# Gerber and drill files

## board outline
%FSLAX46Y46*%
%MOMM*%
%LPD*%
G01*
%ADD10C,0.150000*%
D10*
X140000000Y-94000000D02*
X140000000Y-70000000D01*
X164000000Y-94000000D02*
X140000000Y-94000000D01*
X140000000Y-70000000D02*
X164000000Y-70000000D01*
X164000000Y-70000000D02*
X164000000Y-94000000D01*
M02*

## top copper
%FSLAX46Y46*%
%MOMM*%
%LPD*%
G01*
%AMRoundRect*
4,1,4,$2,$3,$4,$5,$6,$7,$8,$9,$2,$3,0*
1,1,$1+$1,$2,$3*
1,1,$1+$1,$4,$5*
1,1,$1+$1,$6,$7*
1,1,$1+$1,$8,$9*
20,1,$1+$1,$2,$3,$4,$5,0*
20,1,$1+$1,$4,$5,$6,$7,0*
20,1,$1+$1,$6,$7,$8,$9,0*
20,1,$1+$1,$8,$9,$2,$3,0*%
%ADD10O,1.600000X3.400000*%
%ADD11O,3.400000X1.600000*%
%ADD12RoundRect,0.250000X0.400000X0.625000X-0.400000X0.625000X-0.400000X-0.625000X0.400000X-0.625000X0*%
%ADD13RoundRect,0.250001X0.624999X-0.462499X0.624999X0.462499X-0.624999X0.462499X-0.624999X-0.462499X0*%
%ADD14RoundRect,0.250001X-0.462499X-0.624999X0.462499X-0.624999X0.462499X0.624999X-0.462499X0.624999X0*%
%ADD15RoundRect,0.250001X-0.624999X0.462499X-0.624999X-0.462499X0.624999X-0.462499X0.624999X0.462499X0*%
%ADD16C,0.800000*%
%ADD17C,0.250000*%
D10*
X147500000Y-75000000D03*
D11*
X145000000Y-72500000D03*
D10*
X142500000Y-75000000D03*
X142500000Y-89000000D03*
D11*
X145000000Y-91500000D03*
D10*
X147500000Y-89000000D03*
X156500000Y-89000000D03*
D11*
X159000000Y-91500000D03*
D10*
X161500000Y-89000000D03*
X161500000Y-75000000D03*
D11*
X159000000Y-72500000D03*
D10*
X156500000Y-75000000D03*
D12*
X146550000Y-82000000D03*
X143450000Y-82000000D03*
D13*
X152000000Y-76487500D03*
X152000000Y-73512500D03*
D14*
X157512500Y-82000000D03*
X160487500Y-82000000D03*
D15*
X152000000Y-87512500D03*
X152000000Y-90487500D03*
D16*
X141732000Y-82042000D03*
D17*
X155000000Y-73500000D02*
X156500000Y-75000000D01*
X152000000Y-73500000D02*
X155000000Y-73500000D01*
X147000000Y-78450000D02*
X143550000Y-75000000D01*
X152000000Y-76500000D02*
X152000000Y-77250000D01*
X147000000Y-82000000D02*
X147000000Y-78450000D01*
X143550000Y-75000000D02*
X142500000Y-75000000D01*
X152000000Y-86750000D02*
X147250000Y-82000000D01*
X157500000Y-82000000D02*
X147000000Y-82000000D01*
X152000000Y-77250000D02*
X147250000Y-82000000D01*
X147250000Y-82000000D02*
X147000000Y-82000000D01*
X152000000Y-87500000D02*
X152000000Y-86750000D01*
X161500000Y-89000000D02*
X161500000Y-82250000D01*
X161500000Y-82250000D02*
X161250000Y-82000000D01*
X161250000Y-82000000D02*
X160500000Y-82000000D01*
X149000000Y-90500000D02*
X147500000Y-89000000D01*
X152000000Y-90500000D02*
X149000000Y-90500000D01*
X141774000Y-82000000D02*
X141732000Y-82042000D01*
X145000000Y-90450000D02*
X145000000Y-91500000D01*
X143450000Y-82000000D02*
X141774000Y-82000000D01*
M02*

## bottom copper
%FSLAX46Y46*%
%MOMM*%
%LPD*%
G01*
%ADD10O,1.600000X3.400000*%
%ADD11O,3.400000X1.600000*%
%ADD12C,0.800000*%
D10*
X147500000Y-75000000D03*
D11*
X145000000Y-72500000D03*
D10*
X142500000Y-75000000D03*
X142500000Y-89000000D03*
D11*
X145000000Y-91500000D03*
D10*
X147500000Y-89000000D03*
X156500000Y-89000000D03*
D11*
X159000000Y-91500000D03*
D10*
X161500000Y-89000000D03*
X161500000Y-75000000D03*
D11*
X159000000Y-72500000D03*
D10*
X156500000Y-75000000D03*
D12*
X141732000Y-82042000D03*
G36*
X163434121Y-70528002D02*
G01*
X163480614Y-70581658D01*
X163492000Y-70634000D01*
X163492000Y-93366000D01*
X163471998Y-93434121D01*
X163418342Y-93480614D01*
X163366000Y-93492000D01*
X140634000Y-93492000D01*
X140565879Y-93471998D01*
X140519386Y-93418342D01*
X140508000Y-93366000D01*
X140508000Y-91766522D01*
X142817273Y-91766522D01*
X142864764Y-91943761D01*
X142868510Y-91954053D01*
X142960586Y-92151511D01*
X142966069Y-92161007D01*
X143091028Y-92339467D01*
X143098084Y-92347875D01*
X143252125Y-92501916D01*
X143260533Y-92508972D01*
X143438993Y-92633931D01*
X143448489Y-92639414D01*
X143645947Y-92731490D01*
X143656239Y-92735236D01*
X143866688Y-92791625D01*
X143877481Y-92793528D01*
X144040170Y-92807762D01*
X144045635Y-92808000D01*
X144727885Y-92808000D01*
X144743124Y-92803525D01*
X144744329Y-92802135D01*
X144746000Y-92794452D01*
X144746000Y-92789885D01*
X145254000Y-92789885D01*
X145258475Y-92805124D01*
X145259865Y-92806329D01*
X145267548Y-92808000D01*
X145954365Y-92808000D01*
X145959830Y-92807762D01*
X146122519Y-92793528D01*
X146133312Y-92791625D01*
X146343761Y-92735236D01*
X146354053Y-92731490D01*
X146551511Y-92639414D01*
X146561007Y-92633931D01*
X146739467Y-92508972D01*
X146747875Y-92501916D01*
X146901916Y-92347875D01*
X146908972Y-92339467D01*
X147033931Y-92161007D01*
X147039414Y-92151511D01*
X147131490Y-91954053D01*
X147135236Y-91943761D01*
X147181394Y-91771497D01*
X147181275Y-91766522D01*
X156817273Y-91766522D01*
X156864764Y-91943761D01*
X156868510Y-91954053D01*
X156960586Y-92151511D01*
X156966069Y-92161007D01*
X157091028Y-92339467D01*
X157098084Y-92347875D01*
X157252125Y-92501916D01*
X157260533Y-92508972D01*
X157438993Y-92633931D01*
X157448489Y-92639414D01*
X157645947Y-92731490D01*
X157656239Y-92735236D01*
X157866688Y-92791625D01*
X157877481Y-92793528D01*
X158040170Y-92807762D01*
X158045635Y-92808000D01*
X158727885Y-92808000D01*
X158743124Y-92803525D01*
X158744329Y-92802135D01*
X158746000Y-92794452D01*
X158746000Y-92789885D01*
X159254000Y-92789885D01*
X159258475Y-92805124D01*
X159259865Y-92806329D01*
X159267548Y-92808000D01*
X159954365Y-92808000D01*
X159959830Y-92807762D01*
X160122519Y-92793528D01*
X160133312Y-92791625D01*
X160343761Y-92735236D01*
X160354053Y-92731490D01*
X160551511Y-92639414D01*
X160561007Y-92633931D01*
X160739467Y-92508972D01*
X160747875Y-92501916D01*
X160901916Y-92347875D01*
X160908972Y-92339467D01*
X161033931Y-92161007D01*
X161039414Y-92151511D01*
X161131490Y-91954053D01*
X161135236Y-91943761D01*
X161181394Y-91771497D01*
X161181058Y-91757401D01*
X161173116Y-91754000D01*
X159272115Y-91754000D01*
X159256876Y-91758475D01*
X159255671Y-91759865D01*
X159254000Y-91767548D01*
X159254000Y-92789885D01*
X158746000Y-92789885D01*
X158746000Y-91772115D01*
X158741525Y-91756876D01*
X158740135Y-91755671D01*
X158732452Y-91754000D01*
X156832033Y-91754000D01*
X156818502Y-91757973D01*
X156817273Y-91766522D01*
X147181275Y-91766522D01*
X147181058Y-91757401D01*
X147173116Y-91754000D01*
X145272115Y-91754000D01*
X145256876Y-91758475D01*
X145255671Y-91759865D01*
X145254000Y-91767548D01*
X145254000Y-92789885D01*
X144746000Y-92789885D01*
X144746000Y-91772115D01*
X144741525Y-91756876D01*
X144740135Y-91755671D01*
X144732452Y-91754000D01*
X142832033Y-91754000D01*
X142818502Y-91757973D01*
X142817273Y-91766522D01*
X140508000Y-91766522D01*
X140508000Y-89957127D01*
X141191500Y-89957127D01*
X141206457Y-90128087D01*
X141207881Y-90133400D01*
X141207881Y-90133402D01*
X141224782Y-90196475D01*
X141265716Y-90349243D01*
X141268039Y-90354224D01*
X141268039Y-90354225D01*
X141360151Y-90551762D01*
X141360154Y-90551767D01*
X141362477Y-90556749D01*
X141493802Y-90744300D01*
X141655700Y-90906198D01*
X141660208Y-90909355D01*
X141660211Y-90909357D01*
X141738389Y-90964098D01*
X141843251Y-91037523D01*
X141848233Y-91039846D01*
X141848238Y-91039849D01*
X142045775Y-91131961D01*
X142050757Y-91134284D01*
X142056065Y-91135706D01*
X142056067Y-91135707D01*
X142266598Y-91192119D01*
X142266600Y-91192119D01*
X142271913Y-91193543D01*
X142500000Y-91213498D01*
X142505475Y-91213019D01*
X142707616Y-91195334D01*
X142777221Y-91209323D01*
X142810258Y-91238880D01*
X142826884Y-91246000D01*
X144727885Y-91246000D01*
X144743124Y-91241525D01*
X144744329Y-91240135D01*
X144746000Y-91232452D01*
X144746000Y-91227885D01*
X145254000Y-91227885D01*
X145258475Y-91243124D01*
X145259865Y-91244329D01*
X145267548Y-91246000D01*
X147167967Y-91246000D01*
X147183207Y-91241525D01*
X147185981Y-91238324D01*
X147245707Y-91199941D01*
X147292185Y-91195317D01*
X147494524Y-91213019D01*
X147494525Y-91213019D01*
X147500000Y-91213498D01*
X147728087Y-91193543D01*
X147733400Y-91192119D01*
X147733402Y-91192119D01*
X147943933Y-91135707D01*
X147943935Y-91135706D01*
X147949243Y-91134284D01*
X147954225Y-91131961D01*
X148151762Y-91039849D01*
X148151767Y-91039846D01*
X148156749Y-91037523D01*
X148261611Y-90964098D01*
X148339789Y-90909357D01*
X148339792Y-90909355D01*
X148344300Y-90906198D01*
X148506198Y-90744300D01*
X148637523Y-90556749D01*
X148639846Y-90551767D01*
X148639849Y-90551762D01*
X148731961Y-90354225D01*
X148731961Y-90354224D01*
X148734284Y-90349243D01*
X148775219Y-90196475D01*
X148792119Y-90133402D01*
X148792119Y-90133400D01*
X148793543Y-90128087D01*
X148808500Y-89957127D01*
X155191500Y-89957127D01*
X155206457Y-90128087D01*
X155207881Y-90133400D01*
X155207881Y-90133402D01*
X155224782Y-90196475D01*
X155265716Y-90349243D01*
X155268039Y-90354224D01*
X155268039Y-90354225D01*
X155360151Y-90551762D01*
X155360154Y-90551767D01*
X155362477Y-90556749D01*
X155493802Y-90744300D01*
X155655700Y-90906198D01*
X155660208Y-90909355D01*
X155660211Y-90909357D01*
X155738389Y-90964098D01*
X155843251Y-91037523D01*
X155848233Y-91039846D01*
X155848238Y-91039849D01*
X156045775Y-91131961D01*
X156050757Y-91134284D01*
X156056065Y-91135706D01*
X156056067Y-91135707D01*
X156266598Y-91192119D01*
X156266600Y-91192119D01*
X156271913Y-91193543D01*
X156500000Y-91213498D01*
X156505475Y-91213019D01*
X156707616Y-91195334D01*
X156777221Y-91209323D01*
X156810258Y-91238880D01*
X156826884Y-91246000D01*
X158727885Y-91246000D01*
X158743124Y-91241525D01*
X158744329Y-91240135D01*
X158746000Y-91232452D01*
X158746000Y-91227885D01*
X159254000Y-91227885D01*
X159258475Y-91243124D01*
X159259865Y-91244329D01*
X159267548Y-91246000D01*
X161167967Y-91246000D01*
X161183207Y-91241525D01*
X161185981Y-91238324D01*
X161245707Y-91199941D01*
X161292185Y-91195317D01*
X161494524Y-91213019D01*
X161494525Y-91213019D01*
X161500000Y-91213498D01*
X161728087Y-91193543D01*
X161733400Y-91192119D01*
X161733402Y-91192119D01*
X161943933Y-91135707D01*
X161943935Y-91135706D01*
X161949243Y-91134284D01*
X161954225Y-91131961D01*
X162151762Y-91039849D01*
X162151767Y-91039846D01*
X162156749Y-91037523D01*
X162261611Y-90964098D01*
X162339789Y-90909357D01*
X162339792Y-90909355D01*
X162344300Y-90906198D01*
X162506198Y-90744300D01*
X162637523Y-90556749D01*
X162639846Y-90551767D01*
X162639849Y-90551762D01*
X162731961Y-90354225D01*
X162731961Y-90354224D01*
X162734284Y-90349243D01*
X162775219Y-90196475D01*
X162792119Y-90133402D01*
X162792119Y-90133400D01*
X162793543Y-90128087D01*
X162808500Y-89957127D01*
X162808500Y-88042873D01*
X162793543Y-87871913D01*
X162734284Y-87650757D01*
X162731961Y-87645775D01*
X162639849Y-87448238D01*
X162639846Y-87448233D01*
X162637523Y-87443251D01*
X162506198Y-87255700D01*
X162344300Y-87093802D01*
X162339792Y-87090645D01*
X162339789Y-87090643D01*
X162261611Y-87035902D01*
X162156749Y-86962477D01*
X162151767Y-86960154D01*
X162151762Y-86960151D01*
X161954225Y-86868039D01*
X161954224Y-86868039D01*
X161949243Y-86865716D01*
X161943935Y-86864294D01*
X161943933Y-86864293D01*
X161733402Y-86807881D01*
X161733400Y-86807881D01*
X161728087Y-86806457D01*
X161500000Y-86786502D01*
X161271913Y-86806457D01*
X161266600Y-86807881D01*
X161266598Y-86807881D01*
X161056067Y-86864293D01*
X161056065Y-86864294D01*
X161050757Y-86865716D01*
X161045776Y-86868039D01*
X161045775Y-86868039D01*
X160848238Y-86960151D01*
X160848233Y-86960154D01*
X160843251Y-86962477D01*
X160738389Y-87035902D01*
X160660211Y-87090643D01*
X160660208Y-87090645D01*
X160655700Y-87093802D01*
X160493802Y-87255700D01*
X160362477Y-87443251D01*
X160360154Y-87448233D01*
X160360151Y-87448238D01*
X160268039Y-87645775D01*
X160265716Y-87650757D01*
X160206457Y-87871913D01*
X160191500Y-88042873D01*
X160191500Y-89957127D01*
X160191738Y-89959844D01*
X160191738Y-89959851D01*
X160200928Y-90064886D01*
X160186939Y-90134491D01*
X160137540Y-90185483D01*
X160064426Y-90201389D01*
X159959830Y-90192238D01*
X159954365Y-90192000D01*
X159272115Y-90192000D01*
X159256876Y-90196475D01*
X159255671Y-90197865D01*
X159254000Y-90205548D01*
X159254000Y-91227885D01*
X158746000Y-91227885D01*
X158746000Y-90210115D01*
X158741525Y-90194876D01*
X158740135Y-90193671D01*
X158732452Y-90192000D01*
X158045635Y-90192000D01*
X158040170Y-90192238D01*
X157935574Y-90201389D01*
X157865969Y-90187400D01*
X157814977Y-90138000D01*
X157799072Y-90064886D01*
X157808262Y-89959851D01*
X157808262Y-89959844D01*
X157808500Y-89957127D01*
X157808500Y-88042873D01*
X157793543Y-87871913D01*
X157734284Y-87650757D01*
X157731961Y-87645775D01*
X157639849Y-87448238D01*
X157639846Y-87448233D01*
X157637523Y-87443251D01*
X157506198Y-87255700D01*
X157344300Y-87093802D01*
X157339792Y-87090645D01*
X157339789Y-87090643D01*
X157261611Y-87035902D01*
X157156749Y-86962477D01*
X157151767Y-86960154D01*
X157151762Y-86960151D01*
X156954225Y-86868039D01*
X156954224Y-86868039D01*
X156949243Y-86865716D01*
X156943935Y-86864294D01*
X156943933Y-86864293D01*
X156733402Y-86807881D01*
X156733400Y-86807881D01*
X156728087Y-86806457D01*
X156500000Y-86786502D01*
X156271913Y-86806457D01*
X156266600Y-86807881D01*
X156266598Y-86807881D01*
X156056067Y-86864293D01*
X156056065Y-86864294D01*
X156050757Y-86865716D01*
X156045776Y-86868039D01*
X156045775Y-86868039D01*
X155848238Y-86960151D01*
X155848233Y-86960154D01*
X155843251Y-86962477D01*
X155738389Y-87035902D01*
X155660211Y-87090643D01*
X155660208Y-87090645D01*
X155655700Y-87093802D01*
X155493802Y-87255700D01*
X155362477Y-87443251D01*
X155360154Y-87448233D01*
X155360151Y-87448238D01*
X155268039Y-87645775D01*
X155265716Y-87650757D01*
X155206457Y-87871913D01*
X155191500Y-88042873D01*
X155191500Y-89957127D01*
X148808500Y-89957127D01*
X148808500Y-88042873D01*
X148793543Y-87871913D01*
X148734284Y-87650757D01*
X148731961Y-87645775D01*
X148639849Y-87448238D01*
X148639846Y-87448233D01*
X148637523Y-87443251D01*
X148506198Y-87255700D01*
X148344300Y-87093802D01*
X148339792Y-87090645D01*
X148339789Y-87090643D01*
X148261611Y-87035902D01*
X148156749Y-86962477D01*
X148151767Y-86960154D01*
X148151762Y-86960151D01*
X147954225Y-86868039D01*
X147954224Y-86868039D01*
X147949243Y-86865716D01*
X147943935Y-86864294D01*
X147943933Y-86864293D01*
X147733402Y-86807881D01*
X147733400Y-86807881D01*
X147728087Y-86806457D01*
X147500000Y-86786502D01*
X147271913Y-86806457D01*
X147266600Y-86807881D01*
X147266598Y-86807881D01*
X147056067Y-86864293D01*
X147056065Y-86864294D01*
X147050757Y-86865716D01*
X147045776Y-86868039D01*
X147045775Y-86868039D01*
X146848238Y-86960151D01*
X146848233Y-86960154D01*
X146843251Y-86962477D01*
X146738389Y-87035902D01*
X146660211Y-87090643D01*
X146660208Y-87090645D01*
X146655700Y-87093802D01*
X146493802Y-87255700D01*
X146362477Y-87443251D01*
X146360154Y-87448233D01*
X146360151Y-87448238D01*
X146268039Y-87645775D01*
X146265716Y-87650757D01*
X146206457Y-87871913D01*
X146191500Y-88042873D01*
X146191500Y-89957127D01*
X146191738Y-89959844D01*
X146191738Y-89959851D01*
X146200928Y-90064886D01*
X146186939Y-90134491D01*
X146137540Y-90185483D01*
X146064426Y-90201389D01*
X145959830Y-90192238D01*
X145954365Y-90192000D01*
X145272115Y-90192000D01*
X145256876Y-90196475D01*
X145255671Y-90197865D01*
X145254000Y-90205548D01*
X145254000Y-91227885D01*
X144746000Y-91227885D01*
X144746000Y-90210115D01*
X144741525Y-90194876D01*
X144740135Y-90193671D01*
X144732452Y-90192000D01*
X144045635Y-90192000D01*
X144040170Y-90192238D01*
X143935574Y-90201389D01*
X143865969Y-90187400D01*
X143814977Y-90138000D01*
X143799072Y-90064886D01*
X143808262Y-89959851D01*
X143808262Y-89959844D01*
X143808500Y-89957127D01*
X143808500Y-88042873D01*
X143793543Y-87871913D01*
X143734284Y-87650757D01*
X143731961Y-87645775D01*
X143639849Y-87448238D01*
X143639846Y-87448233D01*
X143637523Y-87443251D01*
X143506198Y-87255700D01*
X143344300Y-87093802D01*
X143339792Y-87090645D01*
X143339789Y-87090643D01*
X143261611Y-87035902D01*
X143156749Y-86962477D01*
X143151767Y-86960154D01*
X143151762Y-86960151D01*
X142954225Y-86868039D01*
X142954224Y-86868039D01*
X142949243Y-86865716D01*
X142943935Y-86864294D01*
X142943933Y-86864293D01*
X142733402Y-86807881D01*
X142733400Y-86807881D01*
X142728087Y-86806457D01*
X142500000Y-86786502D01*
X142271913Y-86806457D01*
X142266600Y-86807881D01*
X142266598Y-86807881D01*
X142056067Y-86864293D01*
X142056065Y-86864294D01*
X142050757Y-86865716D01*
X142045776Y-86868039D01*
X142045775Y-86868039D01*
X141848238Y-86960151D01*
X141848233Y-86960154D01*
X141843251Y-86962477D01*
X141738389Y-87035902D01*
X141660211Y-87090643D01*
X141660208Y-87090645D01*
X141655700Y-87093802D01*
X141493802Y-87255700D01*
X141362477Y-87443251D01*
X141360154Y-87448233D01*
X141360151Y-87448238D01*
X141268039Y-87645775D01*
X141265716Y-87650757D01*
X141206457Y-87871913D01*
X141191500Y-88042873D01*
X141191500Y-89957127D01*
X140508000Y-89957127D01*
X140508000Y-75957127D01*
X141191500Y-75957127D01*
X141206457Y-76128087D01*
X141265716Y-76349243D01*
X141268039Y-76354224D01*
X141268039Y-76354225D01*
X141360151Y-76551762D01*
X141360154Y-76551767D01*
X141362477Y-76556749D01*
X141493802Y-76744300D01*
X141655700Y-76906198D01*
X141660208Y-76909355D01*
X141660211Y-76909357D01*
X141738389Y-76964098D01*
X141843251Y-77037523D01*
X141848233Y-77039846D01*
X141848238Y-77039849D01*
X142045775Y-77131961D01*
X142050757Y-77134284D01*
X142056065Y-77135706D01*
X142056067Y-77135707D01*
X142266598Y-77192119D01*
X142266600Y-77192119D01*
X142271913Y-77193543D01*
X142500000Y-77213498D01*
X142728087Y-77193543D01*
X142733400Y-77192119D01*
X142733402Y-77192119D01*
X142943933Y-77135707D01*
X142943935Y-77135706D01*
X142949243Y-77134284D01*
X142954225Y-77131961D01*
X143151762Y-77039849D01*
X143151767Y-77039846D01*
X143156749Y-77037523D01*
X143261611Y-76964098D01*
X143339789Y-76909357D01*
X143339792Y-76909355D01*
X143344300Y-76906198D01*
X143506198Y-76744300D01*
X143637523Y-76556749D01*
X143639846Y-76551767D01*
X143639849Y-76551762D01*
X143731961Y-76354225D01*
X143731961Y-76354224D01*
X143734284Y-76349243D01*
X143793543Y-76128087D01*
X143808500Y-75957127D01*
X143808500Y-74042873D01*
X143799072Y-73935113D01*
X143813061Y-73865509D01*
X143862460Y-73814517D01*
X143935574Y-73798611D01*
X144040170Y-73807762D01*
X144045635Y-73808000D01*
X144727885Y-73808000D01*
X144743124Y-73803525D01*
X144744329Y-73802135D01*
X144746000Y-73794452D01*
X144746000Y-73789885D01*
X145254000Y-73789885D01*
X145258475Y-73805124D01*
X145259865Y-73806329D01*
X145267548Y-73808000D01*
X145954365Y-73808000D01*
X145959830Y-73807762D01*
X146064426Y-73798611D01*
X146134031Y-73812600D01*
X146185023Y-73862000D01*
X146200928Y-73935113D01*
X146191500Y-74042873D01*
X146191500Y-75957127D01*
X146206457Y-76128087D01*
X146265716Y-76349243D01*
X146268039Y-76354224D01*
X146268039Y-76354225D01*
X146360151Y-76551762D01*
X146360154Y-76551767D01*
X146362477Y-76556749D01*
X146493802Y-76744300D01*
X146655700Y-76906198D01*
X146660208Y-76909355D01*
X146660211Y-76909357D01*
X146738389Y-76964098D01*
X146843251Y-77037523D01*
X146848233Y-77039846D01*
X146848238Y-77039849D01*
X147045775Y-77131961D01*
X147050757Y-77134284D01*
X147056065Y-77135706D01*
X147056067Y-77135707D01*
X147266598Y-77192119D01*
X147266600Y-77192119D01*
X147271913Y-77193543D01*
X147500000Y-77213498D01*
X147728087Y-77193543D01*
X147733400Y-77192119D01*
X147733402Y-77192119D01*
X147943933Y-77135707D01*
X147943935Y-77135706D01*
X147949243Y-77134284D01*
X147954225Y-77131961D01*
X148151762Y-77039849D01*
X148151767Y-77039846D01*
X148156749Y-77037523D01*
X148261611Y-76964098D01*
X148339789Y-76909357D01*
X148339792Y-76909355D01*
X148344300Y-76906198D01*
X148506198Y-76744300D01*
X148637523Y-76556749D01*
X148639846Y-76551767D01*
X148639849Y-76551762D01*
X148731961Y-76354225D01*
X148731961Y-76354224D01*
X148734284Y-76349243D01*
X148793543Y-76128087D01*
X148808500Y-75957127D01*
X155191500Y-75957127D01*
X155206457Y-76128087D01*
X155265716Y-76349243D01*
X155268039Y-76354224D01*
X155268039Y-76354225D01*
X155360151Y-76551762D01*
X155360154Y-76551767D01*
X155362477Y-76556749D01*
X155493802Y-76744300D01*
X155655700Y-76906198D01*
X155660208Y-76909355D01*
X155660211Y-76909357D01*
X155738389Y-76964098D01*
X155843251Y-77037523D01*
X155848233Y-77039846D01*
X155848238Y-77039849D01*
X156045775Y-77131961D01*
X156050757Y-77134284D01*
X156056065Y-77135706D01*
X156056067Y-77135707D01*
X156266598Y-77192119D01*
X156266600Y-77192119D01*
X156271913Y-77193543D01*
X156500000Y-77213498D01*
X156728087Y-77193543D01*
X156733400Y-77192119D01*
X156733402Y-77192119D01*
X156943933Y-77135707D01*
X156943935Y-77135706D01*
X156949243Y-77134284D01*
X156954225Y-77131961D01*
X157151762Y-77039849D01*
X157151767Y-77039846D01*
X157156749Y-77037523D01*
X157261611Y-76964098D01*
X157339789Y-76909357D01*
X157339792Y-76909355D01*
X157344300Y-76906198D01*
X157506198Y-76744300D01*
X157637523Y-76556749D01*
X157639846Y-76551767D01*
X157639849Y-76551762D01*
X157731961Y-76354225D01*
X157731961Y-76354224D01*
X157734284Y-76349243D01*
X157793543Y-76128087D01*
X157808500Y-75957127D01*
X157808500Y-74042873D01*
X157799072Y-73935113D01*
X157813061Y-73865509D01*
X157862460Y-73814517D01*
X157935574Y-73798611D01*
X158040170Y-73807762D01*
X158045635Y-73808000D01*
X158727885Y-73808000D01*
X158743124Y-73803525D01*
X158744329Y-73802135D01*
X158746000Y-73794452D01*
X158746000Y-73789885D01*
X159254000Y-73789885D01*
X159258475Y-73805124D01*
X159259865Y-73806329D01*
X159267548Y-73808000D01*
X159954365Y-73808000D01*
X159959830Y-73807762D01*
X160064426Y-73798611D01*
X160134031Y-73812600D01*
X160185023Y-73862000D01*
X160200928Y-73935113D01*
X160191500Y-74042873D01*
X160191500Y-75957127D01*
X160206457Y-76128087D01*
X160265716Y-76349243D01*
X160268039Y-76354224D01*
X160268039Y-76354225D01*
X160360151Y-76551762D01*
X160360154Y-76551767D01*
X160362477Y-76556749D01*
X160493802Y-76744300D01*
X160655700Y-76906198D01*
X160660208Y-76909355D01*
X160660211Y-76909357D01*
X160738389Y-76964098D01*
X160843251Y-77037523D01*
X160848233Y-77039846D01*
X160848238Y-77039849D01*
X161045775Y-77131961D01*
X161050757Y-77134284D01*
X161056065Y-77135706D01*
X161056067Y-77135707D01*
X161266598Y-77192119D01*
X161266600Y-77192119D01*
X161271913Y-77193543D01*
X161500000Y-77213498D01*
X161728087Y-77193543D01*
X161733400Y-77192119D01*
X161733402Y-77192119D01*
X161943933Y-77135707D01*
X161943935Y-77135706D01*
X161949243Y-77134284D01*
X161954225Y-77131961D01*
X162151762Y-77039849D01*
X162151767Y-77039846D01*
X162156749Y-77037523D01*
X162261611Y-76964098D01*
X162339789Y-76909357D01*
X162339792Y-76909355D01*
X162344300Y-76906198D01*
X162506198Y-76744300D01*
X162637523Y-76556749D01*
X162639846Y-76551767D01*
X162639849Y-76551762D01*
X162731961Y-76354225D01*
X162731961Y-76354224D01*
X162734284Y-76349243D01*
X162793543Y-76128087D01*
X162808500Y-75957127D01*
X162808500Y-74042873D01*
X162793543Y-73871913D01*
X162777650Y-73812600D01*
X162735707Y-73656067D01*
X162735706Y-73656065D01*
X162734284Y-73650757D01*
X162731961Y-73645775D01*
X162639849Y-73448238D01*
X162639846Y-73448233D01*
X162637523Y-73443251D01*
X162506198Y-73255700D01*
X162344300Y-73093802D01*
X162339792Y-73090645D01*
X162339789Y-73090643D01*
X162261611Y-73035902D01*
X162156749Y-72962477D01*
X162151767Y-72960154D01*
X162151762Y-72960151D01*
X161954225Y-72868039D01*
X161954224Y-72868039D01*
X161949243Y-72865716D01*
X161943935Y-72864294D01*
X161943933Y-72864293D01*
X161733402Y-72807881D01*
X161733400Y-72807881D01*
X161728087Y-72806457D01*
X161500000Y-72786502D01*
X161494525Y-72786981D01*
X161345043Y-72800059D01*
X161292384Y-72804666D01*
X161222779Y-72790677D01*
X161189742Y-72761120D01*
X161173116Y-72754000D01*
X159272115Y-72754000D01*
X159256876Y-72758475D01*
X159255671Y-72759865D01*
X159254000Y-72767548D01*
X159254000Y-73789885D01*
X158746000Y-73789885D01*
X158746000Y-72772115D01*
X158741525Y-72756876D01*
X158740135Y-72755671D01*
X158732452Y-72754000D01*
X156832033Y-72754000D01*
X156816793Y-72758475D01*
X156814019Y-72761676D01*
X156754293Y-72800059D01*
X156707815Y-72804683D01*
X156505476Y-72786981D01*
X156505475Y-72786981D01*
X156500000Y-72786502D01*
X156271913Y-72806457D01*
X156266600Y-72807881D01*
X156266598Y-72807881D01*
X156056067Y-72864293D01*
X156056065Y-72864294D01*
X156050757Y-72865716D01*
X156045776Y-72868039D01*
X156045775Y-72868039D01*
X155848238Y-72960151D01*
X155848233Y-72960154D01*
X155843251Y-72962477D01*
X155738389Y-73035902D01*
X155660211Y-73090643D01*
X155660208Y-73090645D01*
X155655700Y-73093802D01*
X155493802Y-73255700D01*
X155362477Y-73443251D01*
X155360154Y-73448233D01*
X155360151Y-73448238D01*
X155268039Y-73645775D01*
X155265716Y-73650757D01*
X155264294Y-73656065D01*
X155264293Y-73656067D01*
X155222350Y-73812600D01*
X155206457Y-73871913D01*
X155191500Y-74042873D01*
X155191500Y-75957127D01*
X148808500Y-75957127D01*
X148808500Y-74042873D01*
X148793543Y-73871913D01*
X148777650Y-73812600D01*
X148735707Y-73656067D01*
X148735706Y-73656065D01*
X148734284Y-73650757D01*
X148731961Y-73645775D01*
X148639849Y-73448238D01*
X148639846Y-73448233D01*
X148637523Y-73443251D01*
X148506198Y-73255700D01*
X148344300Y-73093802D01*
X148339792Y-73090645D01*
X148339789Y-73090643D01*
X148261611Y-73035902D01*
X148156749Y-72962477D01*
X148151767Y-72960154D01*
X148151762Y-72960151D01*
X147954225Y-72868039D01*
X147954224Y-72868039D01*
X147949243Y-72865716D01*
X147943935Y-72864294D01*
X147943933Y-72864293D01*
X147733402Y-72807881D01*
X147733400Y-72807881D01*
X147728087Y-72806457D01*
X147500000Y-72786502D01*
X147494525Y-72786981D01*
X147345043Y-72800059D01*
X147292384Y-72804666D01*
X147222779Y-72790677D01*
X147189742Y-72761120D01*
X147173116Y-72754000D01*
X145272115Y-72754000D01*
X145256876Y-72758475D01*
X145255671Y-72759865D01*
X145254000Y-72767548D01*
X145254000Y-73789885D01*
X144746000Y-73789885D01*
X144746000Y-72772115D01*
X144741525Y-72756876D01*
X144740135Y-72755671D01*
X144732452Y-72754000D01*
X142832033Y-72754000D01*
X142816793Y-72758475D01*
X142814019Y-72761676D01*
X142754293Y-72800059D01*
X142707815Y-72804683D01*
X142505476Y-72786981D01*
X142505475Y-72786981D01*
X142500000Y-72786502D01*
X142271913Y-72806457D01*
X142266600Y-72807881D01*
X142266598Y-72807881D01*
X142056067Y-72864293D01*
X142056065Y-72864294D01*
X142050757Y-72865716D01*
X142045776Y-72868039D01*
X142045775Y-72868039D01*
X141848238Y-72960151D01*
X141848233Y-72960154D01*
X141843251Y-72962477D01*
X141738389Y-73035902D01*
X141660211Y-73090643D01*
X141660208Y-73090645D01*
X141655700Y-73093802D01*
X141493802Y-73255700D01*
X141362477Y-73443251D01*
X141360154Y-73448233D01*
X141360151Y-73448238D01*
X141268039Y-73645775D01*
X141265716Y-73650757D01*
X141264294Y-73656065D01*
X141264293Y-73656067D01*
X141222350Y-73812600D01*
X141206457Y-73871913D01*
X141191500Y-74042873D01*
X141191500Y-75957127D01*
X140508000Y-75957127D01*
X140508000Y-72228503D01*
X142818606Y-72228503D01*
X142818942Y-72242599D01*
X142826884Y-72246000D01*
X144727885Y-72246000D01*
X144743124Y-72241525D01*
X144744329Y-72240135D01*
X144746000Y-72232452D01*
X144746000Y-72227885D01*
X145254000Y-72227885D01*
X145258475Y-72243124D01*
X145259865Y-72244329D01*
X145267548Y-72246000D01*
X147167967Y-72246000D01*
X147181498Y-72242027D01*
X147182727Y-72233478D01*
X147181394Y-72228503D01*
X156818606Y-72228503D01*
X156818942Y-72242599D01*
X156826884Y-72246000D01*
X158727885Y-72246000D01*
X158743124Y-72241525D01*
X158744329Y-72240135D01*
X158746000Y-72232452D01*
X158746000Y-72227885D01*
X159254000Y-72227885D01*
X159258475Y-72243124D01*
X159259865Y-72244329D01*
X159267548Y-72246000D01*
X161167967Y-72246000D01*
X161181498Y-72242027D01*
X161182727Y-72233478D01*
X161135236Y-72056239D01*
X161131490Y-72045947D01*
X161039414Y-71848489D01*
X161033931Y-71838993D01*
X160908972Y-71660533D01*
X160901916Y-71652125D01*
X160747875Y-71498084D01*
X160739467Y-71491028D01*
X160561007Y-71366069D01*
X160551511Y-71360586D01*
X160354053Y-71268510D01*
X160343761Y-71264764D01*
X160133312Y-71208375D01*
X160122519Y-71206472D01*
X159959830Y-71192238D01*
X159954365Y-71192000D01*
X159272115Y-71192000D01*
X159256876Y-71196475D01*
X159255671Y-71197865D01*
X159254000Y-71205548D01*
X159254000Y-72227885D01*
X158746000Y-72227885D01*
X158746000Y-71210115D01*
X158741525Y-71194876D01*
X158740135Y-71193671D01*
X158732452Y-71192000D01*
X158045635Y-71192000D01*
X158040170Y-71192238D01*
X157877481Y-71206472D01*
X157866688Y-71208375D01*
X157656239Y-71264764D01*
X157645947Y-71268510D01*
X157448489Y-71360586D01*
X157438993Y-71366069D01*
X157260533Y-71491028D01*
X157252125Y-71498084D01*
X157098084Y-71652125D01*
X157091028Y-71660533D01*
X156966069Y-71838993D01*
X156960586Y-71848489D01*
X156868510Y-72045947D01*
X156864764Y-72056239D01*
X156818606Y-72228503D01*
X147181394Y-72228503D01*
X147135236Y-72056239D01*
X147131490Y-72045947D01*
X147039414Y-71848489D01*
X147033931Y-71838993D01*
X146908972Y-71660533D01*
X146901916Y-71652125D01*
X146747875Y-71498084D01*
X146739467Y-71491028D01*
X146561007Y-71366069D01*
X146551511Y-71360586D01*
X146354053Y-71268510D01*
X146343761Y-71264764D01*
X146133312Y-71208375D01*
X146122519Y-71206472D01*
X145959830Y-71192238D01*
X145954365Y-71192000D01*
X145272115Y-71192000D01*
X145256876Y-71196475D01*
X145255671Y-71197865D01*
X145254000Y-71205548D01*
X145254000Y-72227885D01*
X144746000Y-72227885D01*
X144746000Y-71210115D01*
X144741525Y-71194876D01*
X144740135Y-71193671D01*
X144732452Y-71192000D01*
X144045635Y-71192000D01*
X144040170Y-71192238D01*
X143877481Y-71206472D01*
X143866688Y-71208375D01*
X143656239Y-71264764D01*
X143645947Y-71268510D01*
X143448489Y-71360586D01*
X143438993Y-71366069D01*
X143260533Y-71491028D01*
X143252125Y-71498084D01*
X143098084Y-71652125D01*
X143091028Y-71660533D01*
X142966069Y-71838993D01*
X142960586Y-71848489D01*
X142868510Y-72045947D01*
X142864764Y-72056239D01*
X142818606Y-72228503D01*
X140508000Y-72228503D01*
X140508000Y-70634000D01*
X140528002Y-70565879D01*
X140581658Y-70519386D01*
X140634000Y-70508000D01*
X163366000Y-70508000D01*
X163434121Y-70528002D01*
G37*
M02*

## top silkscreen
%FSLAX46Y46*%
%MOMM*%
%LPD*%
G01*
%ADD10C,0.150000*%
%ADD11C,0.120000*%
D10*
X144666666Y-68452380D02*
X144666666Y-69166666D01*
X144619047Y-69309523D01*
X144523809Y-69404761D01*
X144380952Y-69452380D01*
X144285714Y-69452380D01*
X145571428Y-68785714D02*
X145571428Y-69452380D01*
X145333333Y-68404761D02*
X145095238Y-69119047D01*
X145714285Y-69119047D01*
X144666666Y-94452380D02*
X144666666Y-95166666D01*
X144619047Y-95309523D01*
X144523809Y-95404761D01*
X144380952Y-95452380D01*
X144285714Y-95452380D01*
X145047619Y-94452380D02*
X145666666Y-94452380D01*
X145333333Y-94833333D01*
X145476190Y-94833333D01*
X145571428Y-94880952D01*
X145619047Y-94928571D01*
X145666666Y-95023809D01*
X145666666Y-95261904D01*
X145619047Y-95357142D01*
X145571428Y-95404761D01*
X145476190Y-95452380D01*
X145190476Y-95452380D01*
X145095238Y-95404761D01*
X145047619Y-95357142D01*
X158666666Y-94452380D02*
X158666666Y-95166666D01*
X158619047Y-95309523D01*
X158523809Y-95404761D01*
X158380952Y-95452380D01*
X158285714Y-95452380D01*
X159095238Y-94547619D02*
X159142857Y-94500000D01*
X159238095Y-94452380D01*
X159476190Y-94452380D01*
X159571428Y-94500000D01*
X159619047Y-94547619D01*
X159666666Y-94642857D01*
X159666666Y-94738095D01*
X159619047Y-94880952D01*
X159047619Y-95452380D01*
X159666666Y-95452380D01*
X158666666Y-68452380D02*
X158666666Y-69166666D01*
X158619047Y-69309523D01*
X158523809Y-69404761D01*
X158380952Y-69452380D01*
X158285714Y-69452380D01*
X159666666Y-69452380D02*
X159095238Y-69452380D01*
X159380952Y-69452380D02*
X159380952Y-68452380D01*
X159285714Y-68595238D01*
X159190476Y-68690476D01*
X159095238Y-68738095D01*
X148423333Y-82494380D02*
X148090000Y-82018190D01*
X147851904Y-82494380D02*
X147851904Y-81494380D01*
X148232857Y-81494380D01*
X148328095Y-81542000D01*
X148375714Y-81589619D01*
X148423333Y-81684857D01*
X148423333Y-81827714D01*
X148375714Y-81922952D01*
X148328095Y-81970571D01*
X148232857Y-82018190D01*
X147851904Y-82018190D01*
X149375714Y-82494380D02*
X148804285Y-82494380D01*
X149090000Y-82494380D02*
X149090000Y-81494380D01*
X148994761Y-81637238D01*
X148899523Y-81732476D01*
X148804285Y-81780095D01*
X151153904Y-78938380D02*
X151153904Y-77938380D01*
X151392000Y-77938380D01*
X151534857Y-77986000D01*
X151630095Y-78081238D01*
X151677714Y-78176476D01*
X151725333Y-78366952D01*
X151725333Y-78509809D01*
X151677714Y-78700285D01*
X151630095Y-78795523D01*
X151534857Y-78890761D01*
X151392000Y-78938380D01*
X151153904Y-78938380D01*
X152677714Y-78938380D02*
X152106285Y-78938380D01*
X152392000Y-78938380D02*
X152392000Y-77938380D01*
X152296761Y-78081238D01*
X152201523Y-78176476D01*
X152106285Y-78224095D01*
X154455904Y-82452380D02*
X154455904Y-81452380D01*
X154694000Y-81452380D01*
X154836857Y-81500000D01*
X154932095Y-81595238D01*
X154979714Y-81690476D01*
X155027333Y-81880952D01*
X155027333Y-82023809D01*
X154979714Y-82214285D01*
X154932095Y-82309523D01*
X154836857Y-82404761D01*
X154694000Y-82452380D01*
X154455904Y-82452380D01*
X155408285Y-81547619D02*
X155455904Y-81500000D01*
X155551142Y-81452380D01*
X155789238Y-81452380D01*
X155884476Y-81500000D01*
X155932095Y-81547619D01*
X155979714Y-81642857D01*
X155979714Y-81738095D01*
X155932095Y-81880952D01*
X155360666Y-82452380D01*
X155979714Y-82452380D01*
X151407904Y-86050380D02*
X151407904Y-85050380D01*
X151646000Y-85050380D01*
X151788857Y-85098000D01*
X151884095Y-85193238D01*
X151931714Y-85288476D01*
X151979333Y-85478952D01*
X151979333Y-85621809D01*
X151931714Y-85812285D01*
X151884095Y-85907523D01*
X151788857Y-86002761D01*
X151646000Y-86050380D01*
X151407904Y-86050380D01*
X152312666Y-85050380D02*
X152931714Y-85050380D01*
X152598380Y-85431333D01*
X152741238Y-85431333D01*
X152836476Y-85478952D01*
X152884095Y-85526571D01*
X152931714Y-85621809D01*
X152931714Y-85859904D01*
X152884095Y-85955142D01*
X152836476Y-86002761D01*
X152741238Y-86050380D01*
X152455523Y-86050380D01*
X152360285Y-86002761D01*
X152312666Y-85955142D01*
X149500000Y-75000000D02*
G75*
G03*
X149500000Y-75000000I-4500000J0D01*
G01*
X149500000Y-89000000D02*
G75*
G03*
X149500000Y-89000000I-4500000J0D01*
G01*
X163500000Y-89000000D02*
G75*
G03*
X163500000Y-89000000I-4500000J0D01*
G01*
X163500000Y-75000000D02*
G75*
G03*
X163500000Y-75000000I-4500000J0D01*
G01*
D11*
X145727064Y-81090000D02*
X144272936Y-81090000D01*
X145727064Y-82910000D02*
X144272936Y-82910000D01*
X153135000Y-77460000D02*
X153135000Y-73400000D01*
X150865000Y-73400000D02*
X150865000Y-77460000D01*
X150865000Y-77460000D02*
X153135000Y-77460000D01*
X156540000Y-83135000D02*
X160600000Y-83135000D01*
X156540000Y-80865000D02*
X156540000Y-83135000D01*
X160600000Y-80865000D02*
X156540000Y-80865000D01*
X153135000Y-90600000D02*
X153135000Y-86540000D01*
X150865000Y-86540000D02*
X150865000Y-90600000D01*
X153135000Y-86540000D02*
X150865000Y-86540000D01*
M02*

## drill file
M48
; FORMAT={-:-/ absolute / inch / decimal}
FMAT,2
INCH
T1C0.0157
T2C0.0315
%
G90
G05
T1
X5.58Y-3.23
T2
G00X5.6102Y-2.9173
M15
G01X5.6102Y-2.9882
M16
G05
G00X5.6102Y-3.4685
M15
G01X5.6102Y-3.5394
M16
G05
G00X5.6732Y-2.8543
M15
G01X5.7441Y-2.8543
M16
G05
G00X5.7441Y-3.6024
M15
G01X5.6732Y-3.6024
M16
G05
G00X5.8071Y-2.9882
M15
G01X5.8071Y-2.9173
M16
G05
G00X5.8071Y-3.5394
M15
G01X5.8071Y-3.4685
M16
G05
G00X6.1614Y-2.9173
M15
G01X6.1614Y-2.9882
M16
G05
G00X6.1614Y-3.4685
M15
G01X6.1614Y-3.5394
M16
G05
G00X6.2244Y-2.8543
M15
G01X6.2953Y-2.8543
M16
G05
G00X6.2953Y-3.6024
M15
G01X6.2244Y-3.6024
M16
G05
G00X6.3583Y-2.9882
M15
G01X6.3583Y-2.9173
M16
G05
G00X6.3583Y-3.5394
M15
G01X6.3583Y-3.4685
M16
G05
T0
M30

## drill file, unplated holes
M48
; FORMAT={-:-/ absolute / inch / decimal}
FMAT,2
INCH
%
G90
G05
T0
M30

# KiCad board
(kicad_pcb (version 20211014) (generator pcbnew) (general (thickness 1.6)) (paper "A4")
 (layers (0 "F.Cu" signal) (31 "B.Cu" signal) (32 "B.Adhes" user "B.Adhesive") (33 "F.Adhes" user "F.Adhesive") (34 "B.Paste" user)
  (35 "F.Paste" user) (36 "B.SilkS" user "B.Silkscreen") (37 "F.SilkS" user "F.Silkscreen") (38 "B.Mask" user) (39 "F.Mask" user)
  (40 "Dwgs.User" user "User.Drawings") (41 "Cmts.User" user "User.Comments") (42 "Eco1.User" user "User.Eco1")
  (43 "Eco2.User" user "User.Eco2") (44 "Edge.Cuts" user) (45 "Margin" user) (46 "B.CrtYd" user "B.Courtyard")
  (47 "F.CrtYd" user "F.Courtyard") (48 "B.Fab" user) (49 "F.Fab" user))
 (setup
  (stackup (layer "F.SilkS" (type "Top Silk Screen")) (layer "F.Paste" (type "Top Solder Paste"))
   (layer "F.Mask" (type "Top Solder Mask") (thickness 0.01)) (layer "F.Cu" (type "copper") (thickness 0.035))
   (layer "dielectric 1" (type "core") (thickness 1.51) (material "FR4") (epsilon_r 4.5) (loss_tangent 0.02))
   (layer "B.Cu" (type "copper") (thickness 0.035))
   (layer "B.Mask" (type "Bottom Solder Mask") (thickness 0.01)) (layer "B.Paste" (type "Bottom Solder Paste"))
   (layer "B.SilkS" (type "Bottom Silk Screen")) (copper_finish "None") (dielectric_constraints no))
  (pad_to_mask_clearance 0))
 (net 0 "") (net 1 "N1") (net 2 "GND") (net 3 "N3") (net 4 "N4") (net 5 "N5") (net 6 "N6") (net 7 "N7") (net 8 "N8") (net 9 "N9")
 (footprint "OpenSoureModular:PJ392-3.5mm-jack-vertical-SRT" (layer "F.Cu") (at 145 75)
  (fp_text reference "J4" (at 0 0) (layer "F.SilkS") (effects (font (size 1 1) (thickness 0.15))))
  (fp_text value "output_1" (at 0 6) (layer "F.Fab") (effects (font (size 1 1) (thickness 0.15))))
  (fp_circle (center 0 0) (end 4.5 0) (layer "F.SilkS") (width 0.15) (fill none))
  (pad "R" thru_hole oval locked (at 2.5 0 90) (size 3.4 1.6) (drill oval 2.6 0.8) (layers *.Cu *.Mask) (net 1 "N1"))
  (pad "S" thru_hole oval locked (at 0 -2.5) (size 3.4 1.6) (drill oval 2.6 0.8) (layers *.Cu *.Mask) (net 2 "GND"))
  (pad "T" thru_hole oval locked (at -2.5 0 270) (size 3.4 1.6) (drill oval 2.6 0.8) (layers *.Cu *.Mask) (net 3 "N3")))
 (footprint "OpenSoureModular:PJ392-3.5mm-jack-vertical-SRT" (layer "F.Cu") (at 145 89 180)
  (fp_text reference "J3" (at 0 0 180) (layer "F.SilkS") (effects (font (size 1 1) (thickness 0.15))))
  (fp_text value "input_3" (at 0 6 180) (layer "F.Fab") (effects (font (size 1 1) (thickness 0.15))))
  (fp_circle (center 0 0) (end 4.5 0) (layer "F.SilkS") (width 0.15) (fill none))
  (pad "R" thru_hole oval locked (at 2.5 0 270) (size 3.4 1.6) (drill oval 2.6 0.8) (layers *.Cu *.Mask) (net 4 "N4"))
  (pad "S" thru_hole oval locked (at 0 -2.5 180) (size 3.4 1.6) (drill oval 2.6 0.8) (layers *.Cu *.Mask) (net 2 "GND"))
  (pad "T" thru_hole oval locked (at -2.5 0 90) (size 3.4 1.6) (drill oval 2.6 0.8) (layers *.Cu *.Mask) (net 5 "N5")))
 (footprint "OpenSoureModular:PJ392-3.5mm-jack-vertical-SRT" (layer "F.Cu") (at 159 89 180)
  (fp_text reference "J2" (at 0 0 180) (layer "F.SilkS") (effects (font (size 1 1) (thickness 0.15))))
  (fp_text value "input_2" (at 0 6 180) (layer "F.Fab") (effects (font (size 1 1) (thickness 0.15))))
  (fp_circle (center 0 0) (end 4.5 0) (layer "F.SilkS") (width 0.15) (fill none))
  (pad "R" thru_hole oval locked (at 2.5 0 270) (size 3.4 1.6) (drill oval 2.6 0.8) (layers *.Cu *.Mask) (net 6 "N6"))
  (pad "S" thru_hole oval locked (at 0 -2.5 180) (size 3.4 1.6) (drill oval 2.6 0.8) (layers *.Cu *.Mask) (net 2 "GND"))
  (pad "T" thru_hole oval locked (at -2.5 0 90) (size 3.4 1.6) (drill oval 2.6 0.8) (layers *.Cu *.Mask) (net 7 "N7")))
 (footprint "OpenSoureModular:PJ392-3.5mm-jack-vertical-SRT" (layer "F.Cu") (at 159 75)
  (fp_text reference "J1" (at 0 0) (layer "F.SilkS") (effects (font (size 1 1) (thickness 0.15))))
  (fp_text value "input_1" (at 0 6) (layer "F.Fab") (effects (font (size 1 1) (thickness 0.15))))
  (fp_circle (center 0 0) (end 4.5 0) (layer "F.SilkS") (width 0.15) (fill none))
  (pad "R" thru_hole oval locked (at 2.5 0 90) (size 3.4 1.6) (drill oval 2.6 0.8) (layers *.Cu *.Mask) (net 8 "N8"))
  (pad "S" thru_hole oval locked (at 0 -2.5) (size 3.4 1.6) (drill oval 2.6 0.8) (layers *.Cu *.Mask) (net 2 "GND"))
  (pad "T" thru_hole oval locked (at -2.5 0 270) (size 3.4 1.6) (drill oval 2.6 0.8) (layers *.Cu *.Mask) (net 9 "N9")))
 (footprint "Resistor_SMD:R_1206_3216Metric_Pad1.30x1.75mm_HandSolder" (layer "F.Cu") (at 145 82 180)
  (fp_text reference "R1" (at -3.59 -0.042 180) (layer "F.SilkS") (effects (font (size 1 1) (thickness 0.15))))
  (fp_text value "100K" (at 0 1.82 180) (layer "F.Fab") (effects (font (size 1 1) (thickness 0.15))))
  (fp_line (start -0.727064 0.91) (end 0.727064 0.91) (layer "F.SilkS") (width 0.12))
  (fp_line (start -0.727064 -0.91) (end 0.727064 -0.91) (layer "F.SilkS") (width 0.12))
  (pad "1" smd roundrect (at -1.55 0 180) (size 1.3 1.75) (layers "F.Cu" "F.Paste" "F.Mask") (roundrect_rratio 0.1923076923) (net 3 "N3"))
  (pad "2" smd roundrect (at 1.55 0 180) (size 1.3 1.75) (layers "F.Cu" "F.Paste" "F.Mask") (roundrect_rratio 0.1923076923) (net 2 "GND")))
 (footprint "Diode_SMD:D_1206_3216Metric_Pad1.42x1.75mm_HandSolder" (layer "F.Cu") (at 152 75 90)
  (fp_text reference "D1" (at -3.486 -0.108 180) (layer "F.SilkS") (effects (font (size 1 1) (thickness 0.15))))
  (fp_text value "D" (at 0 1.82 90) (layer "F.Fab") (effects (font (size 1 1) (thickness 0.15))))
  (fp_line (start -2.46 1.135) (end 1.6 1.135) (layer "F.SilkS") (width 0.12))
  (fp_line (start 1.6 -1.135) (end -2.46 -1.135) (layer "F.SilkS") (width 0.12))
  (fp_line (start -2.46 -1.135) (end -2.46 1.135) (layer "F.SilkS") (width 0.12))
  (pad "1" smd roundrect (at -1.4875 0 90) (size 1.425 1.75) (layers "F.Cu" "F.Paste" "F.Mask") (roundrect_rratio 0.1754392982) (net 3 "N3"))
  (pad "2" smd roundrect (at 1.4875 0 90) (size 1.425 1.75) (layers "F.Cu" "F.Paste" "F.Mask") (roundrect_rratio 0.1754392982) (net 9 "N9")))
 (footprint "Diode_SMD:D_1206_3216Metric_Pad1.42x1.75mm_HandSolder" (layer "F.Cu") (at 159 82)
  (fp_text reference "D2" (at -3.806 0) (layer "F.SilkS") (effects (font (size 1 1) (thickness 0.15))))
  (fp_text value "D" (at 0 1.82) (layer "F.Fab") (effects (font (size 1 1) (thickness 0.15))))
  (fp_line (start -2.46 1.135) (end 1.6 1.135) (layer "F.SilkS") (width 0.12))
  (fp_line (start -2.46 -1.135) (end -2.46 1.135) (layer "F.SilkS") (width 0.12))
  (fp_line (start 1.6 -1.135) (end -2.46 -1.135) (layer "F.SilkS") (width 0.12))
  (pad "1" smd roundrect (at -1.4875 0) (size 1.425 1.75) (layers "F.Cu" "F.Paste" "F.Mask") (roundrect_rratio 0.1754392982) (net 3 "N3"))
  (pad "2" smd roundrect (at 1.4875 0) (size 1.425 1.75) (layers "F.Cu" "F.Paste" "F.Mask") (roundrect_rratio 0.1754392982) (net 7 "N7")))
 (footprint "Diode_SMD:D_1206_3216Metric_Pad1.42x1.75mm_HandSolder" (layer "F.Cu") (at 152 89 -90)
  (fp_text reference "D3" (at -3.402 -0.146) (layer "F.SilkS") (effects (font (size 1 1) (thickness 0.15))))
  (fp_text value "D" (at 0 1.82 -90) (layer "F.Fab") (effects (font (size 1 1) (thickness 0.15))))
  (fp_line (start 1.6 -1.135) (end -2.46 -1.135) (layer "F.SilkS") (width 0.12))
  (fp_line (start -2.46 1.135) (end 1.6 1.135) (layer "F.SilkS") (width 0.12))
  (fp_line (start -2.46 -1.135) (end -2.46 1.135) (layer "F.SilkS") (width 0.12))
  (pad "1" smd roundrect (at -1.4875 0 270) (size 1.425 1.75) (layers "F.Cu" "F.Paste" "F.Mask") (roundrect_rratio 0.1754392982)
   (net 3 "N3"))
  (pad "2" smd roundrect (at 1.4875 0 270) (size 1.425 1.75) (layers "F.Cu" "F.Paste" "F.Mask") (roundrect_rratio 0.1754392982) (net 5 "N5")))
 (gr_line (start 140 94) (end 140 70) (layer "Edge.Cuts") (width 0.15))
 (gr_line (start 164 94) (end 140 94) (layer "Edge.Cuts") (width 0.15))
 (gr_line (start 140 70) (end 164 70) (layer "Edge.Cuts") (width 0.15))
 (gr_line (start 164 70) (end 164 94) (layer "Edge.Cuts") (width 0.15))
 (segment (start 155 73.5) (end 156.5 75) (width 0.25) (layer "F.Cu") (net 9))
 (segment (start 152 73.5) (end 155 73.5) (width 0.25) (layer "F.Cu") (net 9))
 (segment (start 147 78.45) (end 143.55 75) (width 0.25) (layer "F.Cu") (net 3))
 (segment (start 152 76.5) (end 152 77.25) (width 0.25) (layer "F.Cu") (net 3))
 (segment (start 147 82) (end 147 78.45) (width 0.25) (layer "F.Cu") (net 3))
 (segment (start 143.55 75) (end 142.5 75) (width 0.25) (layer "F.Cu") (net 3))
 (segment (start 152 86.75) (end 147.25 82) (width 0.25) (layer "F.Cu") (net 3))
 (segment (start 157.5 82) (end 147 82) (width 0.25) (layer "F.Cu") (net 3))
 (segment (start 152 77.25) (end 147.25 82) (width 0.25) (layer "F.Cu") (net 3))
 (segment (start 147.25 82) (end 147 82) (width 0.25) (layer "F.Cu") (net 3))
 (segment (start 152 87.5) (end 152 86.75) (width 0.25) (layer "F.Cu") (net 3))
 (segment (start 161.5 89) (end 161.5 82.25) (width 0.25) (layer "F.Cu") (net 7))
 (segment (start 161.5 82.25) (end 161.25 82) (width 0.25) (layer "F.Cu") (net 7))
 (segment (start 161.25 82) (end 160.5 82) (width 0.25) (layer "F.Cu") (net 7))
 (segment (start 149 90.5) (end 147.5 89) (width 0.25) (layer "F.Cu") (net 5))
 (segment (start 152 90.5) (end 149 90.5) (width 0.25) (layer "F.Cu") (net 5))
 (segment (start 141.774 82) (end 141.732 82.042) (width 0.25) (layer "F.Cu") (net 2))
 (segment (start 145 90.45) (end 145 91.5) (width 0.25) (layer "F.Cu") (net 2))
 (segment (start 143.45 82) (end 141.774 82) (width 0.25) (layer "F.Cu") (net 2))
 (via (at 141.732 82.042) (size 0.8) (drill 0.4) (layers "F.Cu" "B.Cu") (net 2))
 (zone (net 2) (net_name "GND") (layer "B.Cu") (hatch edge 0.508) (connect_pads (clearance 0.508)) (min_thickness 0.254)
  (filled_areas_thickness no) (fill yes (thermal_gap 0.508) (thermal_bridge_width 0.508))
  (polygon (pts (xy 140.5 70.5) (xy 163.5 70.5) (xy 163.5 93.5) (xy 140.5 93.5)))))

